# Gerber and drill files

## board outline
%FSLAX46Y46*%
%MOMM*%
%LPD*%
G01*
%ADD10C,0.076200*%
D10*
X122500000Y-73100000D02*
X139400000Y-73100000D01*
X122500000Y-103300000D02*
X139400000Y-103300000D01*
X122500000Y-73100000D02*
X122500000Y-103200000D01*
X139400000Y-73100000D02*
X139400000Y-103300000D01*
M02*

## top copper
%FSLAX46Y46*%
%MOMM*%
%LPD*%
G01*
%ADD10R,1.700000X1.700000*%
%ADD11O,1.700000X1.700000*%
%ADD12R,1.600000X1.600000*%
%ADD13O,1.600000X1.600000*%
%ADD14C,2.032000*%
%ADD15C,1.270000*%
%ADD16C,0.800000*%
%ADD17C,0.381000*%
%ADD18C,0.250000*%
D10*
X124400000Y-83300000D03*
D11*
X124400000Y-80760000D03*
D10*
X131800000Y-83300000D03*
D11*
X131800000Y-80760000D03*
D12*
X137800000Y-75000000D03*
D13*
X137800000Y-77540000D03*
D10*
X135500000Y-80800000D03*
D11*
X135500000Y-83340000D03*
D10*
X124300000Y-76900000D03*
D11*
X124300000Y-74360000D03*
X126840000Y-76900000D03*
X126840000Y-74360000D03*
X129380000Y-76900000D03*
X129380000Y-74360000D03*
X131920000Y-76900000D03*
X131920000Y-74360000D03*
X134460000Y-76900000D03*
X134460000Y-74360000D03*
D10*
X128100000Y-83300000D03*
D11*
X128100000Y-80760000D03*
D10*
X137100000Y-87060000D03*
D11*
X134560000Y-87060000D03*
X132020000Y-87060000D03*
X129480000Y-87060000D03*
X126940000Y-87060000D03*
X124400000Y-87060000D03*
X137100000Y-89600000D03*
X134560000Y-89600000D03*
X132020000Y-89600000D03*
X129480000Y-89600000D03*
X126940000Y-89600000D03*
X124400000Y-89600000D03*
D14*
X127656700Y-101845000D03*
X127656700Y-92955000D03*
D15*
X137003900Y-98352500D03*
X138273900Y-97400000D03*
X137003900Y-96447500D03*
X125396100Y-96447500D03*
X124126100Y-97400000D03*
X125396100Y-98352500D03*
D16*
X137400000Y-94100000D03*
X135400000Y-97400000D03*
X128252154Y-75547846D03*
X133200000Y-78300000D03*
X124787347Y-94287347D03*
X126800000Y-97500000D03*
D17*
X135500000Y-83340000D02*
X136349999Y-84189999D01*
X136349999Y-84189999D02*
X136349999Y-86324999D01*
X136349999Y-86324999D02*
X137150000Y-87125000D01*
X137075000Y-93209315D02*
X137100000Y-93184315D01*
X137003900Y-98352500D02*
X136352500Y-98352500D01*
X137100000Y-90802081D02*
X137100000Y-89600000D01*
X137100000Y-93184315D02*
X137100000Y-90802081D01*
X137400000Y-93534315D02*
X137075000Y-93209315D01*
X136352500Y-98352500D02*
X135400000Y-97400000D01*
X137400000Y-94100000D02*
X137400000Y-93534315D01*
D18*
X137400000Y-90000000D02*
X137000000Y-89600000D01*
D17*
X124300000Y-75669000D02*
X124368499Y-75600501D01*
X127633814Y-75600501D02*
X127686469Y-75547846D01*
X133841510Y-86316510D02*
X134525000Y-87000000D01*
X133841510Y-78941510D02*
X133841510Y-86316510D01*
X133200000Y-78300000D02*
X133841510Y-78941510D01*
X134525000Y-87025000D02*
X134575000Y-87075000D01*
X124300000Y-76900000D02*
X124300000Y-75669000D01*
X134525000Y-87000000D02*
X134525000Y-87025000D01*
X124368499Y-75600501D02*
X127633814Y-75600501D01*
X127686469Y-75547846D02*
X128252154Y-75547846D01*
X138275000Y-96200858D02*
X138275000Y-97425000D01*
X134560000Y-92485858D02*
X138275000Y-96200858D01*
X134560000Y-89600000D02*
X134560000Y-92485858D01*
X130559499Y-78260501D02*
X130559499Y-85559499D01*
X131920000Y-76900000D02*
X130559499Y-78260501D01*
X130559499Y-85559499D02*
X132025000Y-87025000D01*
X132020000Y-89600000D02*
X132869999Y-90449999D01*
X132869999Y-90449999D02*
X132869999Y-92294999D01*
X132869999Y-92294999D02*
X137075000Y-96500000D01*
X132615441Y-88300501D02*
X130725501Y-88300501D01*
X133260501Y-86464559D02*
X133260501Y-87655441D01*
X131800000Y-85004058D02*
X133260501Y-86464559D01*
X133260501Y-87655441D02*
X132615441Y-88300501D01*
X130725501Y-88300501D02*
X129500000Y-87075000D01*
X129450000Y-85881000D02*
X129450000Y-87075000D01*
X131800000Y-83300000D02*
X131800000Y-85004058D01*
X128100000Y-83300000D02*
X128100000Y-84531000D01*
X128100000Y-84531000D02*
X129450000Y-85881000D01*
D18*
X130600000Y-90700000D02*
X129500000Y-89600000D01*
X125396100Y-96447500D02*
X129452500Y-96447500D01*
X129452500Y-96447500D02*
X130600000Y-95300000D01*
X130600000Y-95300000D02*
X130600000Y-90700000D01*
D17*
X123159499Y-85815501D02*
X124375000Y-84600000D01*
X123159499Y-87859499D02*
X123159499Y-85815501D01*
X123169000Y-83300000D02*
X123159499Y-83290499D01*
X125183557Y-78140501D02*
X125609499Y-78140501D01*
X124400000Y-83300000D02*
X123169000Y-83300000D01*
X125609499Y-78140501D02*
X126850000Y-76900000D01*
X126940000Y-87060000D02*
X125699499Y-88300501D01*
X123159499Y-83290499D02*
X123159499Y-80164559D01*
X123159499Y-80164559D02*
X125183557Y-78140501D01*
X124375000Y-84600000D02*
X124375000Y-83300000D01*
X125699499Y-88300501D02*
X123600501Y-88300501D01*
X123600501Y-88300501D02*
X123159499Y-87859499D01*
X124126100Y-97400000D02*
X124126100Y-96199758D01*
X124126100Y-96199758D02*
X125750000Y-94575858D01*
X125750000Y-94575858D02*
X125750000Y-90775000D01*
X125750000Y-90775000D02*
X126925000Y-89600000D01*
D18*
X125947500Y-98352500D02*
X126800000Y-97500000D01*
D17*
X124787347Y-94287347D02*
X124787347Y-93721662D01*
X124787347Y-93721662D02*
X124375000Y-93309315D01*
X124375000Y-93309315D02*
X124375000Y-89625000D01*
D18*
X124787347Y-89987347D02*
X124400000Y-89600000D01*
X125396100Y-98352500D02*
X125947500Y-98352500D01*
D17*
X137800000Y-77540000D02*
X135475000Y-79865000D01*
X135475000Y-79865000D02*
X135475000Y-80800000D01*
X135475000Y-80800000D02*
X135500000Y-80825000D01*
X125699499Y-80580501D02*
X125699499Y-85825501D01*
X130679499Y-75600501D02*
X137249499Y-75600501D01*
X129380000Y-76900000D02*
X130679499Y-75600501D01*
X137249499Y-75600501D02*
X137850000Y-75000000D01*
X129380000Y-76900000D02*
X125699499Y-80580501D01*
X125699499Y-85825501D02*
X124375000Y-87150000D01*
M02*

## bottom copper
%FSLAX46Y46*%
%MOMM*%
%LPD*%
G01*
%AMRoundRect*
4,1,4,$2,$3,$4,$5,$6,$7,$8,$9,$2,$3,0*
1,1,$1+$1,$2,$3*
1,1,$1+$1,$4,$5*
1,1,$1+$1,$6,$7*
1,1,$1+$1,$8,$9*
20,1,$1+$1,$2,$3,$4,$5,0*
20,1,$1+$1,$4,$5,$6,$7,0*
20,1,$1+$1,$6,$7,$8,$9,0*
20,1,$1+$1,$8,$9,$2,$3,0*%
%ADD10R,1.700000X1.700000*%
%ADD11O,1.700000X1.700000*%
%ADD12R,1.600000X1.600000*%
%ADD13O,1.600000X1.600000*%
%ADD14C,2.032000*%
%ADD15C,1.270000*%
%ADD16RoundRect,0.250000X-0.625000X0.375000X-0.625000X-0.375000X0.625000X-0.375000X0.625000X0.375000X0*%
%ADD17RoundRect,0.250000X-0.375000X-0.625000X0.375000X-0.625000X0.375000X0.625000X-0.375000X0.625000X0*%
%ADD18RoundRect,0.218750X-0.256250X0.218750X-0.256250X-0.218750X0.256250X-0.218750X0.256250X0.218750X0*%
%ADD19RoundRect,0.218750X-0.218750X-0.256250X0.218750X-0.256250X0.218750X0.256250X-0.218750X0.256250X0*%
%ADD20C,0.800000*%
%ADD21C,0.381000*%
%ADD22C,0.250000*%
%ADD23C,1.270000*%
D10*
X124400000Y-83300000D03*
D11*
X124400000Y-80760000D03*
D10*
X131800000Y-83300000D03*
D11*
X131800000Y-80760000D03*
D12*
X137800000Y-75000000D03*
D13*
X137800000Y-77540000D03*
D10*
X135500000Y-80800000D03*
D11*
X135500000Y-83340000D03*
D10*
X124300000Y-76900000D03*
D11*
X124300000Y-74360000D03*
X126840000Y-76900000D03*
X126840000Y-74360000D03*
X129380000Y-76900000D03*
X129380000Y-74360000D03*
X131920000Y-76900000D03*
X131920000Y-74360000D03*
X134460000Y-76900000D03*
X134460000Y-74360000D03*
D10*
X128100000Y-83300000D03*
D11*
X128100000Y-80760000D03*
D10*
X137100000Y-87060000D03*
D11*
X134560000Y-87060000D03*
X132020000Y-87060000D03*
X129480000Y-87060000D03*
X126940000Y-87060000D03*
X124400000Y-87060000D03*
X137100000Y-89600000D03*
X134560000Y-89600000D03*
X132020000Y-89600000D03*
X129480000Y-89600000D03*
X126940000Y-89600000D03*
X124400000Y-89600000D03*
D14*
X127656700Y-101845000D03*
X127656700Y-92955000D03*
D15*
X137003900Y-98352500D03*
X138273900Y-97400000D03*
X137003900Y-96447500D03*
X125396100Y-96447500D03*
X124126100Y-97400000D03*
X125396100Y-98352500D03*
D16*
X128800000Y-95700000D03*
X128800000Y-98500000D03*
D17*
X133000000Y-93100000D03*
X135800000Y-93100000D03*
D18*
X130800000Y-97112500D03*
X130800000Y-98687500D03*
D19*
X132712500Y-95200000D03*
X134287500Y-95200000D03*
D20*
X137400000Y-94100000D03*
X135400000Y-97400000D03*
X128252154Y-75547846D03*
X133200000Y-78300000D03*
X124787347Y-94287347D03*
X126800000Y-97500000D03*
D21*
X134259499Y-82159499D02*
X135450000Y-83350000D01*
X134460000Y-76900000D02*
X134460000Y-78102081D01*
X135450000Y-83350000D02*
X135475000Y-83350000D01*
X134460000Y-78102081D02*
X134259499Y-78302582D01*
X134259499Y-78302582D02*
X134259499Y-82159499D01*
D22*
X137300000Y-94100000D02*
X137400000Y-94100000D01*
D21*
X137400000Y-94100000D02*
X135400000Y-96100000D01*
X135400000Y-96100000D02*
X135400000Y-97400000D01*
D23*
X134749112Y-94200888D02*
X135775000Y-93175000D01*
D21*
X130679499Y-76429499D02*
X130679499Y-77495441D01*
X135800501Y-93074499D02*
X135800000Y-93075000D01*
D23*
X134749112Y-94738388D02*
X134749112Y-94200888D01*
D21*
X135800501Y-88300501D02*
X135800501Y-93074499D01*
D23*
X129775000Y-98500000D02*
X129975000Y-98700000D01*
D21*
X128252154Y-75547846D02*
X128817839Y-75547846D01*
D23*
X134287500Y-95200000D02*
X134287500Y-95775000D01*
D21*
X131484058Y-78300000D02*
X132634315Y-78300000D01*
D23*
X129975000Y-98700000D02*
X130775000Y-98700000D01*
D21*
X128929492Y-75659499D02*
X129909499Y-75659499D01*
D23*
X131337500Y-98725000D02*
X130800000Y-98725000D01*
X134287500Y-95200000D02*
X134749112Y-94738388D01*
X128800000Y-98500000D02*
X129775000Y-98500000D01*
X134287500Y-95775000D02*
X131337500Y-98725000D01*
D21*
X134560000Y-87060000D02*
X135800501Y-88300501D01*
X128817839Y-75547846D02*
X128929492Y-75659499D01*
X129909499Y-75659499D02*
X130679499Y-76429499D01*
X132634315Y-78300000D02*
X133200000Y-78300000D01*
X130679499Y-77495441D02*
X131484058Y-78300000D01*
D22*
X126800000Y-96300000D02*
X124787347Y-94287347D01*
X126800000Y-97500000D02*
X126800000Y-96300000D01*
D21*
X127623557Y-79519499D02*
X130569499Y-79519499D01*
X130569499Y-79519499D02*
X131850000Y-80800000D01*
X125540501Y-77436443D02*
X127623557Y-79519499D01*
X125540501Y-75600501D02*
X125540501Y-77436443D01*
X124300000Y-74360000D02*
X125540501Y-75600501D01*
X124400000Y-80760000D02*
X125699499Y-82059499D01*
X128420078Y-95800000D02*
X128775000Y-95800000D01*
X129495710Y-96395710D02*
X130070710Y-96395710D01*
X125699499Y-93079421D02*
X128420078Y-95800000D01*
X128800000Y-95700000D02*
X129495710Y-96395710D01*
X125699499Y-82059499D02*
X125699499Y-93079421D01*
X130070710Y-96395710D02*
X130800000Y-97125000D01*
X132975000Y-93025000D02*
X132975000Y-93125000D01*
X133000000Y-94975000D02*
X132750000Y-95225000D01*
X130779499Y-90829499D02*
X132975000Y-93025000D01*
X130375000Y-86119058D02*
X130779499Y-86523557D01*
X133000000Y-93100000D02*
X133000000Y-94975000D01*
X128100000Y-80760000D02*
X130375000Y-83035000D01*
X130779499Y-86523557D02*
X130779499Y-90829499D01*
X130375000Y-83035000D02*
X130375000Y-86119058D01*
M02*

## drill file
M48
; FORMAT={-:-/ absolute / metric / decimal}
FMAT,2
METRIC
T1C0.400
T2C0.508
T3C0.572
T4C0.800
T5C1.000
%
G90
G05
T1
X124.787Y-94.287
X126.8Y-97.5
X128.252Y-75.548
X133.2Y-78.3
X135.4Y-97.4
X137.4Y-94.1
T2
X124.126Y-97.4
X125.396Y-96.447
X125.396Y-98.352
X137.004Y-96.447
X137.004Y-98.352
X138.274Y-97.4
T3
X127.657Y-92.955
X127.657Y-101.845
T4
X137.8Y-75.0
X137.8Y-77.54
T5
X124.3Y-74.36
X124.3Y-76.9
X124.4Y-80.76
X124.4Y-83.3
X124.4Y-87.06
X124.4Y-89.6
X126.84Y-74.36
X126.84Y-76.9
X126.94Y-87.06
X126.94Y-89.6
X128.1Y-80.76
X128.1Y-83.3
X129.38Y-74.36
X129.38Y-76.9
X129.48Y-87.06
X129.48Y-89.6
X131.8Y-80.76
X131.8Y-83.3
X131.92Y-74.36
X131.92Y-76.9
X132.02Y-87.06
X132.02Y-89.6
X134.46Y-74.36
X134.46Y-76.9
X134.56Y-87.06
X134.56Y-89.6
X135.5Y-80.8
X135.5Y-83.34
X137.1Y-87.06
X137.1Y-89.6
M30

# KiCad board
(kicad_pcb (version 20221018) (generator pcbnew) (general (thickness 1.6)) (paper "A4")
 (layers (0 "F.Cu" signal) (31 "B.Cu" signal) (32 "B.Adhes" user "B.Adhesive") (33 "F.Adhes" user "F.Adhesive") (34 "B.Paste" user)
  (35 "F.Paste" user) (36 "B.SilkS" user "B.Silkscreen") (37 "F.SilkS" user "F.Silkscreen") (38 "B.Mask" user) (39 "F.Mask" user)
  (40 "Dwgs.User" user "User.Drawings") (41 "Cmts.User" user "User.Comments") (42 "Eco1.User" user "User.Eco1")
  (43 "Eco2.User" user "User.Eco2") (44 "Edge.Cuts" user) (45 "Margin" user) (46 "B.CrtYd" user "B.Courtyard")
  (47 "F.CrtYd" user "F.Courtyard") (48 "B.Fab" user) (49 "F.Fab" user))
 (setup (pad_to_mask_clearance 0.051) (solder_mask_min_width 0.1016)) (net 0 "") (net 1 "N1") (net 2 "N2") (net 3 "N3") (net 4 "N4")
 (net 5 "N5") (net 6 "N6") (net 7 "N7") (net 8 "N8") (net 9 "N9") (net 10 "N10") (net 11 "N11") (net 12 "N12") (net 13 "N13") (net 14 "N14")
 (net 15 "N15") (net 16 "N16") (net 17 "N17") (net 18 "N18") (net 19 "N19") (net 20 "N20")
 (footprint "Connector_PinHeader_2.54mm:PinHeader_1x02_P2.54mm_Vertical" (layer "F.Cu") (at 124.4 83.3 180)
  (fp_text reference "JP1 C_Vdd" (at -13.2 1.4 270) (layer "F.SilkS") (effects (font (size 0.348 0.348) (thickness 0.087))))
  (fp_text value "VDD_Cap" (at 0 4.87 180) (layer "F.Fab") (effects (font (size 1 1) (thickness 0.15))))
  (pad "1" thru_hole rect (at 0 0 180) (size 1.7 1.7) (drill 1) (layers "*.Cu" "*.Mask") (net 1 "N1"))
  (pad "2" thru_hole oval (at 0 2.54 180) (size 1.7 1.7) (drill 1) (layers "*.Cu" "*.Mask") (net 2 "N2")))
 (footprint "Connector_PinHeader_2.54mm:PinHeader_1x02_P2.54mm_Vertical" (layer "F.Cu") (at 131.8 83.3 180)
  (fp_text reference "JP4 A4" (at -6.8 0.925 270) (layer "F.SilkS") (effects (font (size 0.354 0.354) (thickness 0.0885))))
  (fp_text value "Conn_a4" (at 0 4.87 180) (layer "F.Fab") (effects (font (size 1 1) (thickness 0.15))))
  (pad "1" thru_hole rect (at 0 0 180) (size 1.7 1.7) (drill 1) (layers "*.Cu" "*.Mask") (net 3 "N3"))
  (pad "2" thru_hole oval (at 0 2.54 180) (size 1.7 1.7) (drill 1) (layers "*.Cu" "*.Mask") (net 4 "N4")))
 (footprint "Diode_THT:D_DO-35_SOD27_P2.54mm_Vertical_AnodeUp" (layer "F.Cu") (at 137.8 75 -90)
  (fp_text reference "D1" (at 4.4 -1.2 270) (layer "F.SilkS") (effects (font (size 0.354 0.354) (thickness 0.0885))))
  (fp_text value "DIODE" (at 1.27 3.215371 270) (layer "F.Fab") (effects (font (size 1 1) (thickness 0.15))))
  (pad "1" thru_hole rect (at 0 0 270) (size 1.6 1.6) (drill 0.8) (layers "*.Cu" "*.Mask") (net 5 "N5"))
  (pad "2" thru_hole oval (at 2.54 0 270) (size 1.6 1.6) (drill 0.8) (layers "*.Cu" "*.Mask") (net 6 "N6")))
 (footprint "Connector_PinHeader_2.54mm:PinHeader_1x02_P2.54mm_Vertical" (layer "F.Cu") (at 135.5 80.8)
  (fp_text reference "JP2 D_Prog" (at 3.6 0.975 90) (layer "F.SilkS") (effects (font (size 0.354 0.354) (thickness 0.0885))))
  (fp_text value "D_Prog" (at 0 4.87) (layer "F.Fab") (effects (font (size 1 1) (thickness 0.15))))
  (pad "1" thru_hole rect (at 0 0) (size 1.7 1.7) (drill 1) (layers "*.Cu" "*.Mask") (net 6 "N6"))
  (pad "2" thru_hole oval (at 0 2.54) (size 1.7 1.7) (drill 1) (layers "*.Cu" "*.Mask") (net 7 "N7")))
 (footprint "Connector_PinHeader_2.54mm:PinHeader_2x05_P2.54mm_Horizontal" (layer "F.Cu") (at 124.3 76.9 90)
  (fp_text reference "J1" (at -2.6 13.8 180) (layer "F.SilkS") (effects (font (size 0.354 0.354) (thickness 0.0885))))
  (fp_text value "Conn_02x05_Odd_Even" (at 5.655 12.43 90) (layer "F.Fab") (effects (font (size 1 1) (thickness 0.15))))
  (pad "1" thru_hole rect (at 0 0 90) (size 1.7 1.7) (drill 1) (layers "*.Cu" "*.Mask") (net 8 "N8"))
  (pad "2" thru_hole oval (at 2.54 0 90) (size 1.7 1.7) (drill 1) (layers "*.Cu" "*.Mask") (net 4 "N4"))
  (pad "3" thru_hole oval (at 0 2.54 90) (size 1.7 1.7) (drill 1) (layers "*.Cu" "*.Mask") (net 1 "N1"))
  (pad "4" thru_hole oval (at 2.54 2.54 90) (size 1.7 1.7) (drill 1) (layers "*.Cu" "*.Mask") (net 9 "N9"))
  (pad "5" thru_hole oval (at 0 5.08 90) (size 1.7 1.7) (drill 1) (layers "*.Cu" "*.Mask") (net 5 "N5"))
  (pad "6" thru_hole oval (at 2.54 5.08 90) (size 1.7 1.7) (drill 1) (layers "*.Cu" "*.Mask") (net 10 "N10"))
  (pad "7" thru_hole oval (at 0 7.62 90) (size 1.7 1.7) (drill 1) (layers "*.Cu" "*.Mask") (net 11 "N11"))
  (pad "8" thru_hole oval (at 2.54 7.62 90) (size 1.7 1.7) (drill 1) (layers "*.Cu" "*.Mask") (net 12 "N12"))
  (pad "9" thru_hole oval (at 0 10.16 90) (size 1.7 1.7) (drill 1) (layers "*.Cu" "*.Mask") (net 7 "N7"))
  (pad "10" thru_hole oval (at 2.54 10.16 90) (size 1.7 1.7) (drill 1) (layers "*.Cu" "*.Mask") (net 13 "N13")))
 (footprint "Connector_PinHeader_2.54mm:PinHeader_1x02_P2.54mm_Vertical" (layer "F.Cu") (at 128.1 83.3 180)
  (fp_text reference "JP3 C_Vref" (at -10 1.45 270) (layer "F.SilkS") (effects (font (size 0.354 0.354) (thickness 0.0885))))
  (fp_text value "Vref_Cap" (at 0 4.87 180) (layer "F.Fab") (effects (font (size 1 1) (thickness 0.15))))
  (pad "1" thru_hole rect (at 0 0 180) (size 1.7 1.7) (drill 1) (layers "*.Cu" "*.Mask") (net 3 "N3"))
  (pad "2" thru_hole oval (at 0 2.54 180) (size 1.7 1.7) (drill 1) (layers "*.Cu" "*.Mask") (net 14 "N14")))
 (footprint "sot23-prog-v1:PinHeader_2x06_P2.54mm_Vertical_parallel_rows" (layer "F.Cu") (at 137.1 87.06 -90)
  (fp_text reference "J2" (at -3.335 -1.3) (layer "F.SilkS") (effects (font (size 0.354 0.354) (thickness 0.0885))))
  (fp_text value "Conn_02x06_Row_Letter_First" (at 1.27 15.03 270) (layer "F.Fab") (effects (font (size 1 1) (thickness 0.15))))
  (pad "a1" thru_hole rect (at 0 0 270) (size 1.7 1.7) (drill 1) (layers "*.Cu" "*.Mask") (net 7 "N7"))
  (pad "a2" thru_hole oval (at 0 2.54 270) (size 1.7 1.7) (drill 1) (layers "*.Cu" "*.Mask") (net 8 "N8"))
  (pad "a3" thru_hole oval (at 0 5.08 270) (size 1.7 1.7) (drill 1) (layers "*.Cu" "*.Mask") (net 11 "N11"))
  (pad "a4" thru_hole oval (at 0 7.62 270) (size 1.7 1.7) (drill 1) (layers "*.Cu" "*.Mask") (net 3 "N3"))
  (pad "a5" thru_hole oval (at 0 10.16 270) (size 1.7 1.7) (drill 1) (layers "*.Cu" "*.Mask") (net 1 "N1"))
  (pad "a6" thru_hole oval (at 0 12.7 270) (size 1.7 1.7) (drill 1) (layers "*.Cu" "*.Mask") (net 5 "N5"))
  (pad "b1" thru_hole oval (at 2.54 0 270) (size 1.7 1.7) (drill 1) (layers "*.Cu" "*.Mask") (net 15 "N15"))
  (pad "b2" thru_hole oval (at 2.54 2.54 270) (size 1.7 1.7) (drill 1) (layers "*.Cu" "*.Mask") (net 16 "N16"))
  (pad "b3" thru_hole oval (at 2.54 5.08 270) (size 1.7 1.7) (drill 1) (layers "*.Cu" "*.Mask") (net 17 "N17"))
  (pad "b4" thru_hole oval (at 2.54 7.62 270) (size 1.7 1.7) (drill 1) (layers "*.Cu" "*.Mask") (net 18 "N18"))
  (pad "b5" thru_hole oval (at 2.54 10.16 270) (size 1.7 1.7) (drill 1) (layers "*.Cu" "*.Mask") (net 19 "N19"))
  (pad "b6" thru_hole oval (at 2.54 12.7 270) (size 1.7 1.7) (drill 1) (layers "*.Cu" "*.Mask") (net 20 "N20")))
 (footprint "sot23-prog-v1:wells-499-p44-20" (layer "F.Cu") (at 131.2 97.4 90)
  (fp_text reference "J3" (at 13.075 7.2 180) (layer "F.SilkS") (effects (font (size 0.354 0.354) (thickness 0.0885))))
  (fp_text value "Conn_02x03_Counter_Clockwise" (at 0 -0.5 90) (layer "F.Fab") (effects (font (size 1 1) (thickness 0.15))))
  (pad "" thru_hole circle (at -4.445 -3.5433 90) (size 2.032 2.032) (drill 0.5715) (layers "*.Cu" "*.Mask"))
  (pad "" thru_hole circle (at 4.445 -3.5433 90) (size 2.032 2.032) (drill 0.5715) (layers "*.Cu" "*.Mask"))
  (pad "1" thru_hole circle (at -0.9525 5.8039 90) (size 1.27 1.27) (drill 0.508) (layers "*.Cu" "*.Mask") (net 15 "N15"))
  (pad "2" thru_hole circle (at 0 7.0739 90) (size 1.27 1.27) (drill 0.508) (layers "*.Cu" "*.Mask") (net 16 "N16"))
  (pad "3" thru_hole circle (at 0.9525 5.8039 90) (size 1.27 1.27) (drill 0.508) (layers "*.Cu" "*.Mask") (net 17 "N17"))
  (pad "4" thru_hole circle (at 0.9525 -5.8039 90) (size 1.27 1.27) (drill 0.508) (layers "*.Cu" "*.Mask") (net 18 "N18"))
  (pad "5" thru_hole circle (at 0 -7.0739 90) (size 1.27 1.27) (drill 0.508) (layers "*.Cu" "*.Mask") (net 19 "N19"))
  (pad "6" thru_hole circle (at -0.9525 -5.8039 90) (size 1.27 1.27) (drill 0.508) (layers "*.Cu" "*.Mask") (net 20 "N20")))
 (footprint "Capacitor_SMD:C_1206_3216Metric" (layer "B.Cu") (at 128.8 97.1 -90)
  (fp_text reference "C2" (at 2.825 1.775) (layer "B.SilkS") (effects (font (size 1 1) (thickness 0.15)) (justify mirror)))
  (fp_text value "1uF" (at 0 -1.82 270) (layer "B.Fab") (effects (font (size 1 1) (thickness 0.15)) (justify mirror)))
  (pad "1" smd roundrect (at -1.4 0 270) (size 1.25 1.75) (layers "B.Cu" "B.Paste" "B.Mask") (roundrect_rratio 0.2) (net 2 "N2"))
  (pad "2" smd roundrect (at 1.4 0 270) (size 1.25 1.75) (layers "B.Cu" "B.Paste" "B.Mask") (roundrect_rratio 0.2) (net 8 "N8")))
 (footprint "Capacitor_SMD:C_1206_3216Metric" (layer "B.Cu") (at 134.4 93.1)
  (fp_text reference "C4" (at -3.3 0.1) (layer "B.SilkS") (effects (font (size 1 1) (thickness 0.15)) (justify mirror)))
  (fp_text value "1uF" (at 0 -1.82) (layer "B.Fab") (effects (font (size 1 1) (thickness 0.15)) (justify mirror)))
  (pad "1" smd roundrect (at -1.4 0) (size 1.25 1.75) (layers "B.Cu" "B.Paste" "B.Mask") (roundrect_rratio 0.2) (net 14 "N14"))
  (pad "2" smd roundrect (at 1.4 0) (size 1.25 1.75) (layers "B.Cu" "B.Paste" "B.Mask") (roundrect_rratio 0.2) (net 8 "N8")))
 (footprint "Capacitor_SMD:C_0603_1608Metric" (layer "B.Cu") (at 130.8 97.9 -90)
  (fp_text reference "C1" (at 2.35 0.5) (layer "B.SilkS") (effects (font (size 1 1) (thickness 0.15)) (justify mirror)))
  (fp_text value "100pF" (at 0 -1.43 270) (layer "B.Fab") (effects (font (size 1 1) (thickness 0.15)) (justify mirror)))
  (pad "1" smd roundrect (at -0.7875 0 270) (size 0.875 0.95) (layers "B.Cu" "B.Paste" "B.Mask") (roundrect_rratio 0.25) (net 2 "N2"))
  (pad "2" smd roundrect (at 0.7875 0 270) (size 0.875 0.95) (layers "B.Cu" "B.Paste" "B.Mask") (roundrect_rratio 0.25) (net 8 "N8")))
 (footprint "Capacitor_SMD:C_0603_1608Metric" (layer "B.Cu") (at 133.5 95.2)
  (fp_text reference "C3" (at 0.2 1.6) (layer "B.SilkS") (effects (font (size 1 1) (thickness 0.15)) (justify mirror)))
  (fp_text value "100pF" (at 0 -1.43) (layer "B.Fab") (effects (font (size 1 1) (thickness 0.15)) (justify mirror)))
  (pad "1" smd roundrect (at -0.7875 0) (size 0.875 0.95) (layers "B.Cu" "B.Paste" "B.Mask") (roundrect_rratio 0.25) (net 14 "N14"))
  (pad "2" smd roundrect (at 0.7875 0) (size 0.875 0.95) (layers "B.Cu" "B.Paste" "B.Mask") (roundrect_rratio 0.25) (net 8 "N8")))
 (gr_line (start 122.5 73.1) (end 139.4 73.1) (stroke (width 0.0762) (type solid)) (layer "Edge.Cuts"))
 (gr_line (start 122.5 103.3) (end 139.4 103.3) (stroke (width 0.0762) (type solid)) (layer "Edge.Cuts"))
 (gr_line (start 122.5 73.1) (end 122.5 103.2) (stroke (width 0.0762) (type solid)) (layer "Edge.Cuts"))
 (gr_line (start 139.4 73.1) (end 139.4 103.3) (stroke (width 0.0762) (type solid)) (layer "Edge.Cuts"))
 (segment (start 135.5 83.34) (end 136.349999 84.189999) (width 0.381) (layer "F.Cu") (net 7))
 (segment (start 136.349999 84.189999) (end 136.349999 86.324999) (width 0.381) (layer "F.Cu") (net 7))
 (segment (start 136.349999 86.324999) (end 137.15 87.125) (width 0.381) (layer "F.Cu") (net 7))
 (segment (start 134.259499 82.159499) (end 135.45 83.35) (width 0.381) (layer "B.Cu") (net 7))
 (segment (start 134.46 76.9) (end 134.46 78.102081) (width 0.381) (layer "B.Cu") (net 7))
 (segment (start 135.45 83.35) (end 135.475 83.35) (width 0.381) (layer "B.Cu") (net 7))
 (segment (start 134.46 78.102081) (end 134.259499 78.302582) (width 0.381) (layer "B.Cu") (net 7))
 (segment (start 134.259499 78.302582) (end 134.259499 82.159499) (width 0.381) (layer "B.Cu") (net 7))
 (segment (start 137.075 93.209315) (end 137.1 93.184315) (width 0.381) (layer "F.Cu") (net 15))
 (segment (start 137.0039 98.3525) (end 136.3525 98.3525) (width 0.381) (layer "F.Cu") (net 15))
 (segment (start 137.1 90.802081) (end 137.1 89.6) (width 0.381) (layer "F.Cu") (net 15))
 (segment (start 137.1 93.184315) (end 137.1 90.802081) (width 0.381) (layer "F.Cu") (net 15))
 (segment (start 137.4 93.534315) (end 137.075 93.209315) (width 0.381) (layer "F.Cu") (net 15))
 (segment (start 136.3525 98.3525) (end 135.4 97.4) (width 0.381) (layer "F.Cu") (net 15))
 (segment (start 137.4 94.1) (end 137.4 93.534315) (width 0.381) (layer "F.Cu") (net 15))
 (segment (start 137.4 90) (end 137 89.6) (width 0.25) (layer "F.Cu") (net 15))
 (via (at 137.4 94.1) (size 0.8) (drill 0.4) (layers "F.Cu" "B.Cu") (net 15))
 (via (at 135.4 97.4) (size 0.8) (drill 0.4) (layers "F.Cu" "B.Cu") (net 15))
 (segment (start 137.3 94.1) (end 137.4 94.1) (width 0.25) (layer "B.Cu") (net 15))
 (segment (start 137.4 94.1) (end 135.4 96.1) (width 0.381) (layer "B.Cu") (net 15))
 (segment (start 135.4 96.1) (end 135.4 97.4) (width 0.381) (layer "B.Cu") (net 15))
 (segment (start 124.3 75.669) (end 124.368499 75.600501) (width 0.381) (layer "F.Cu") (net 8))
 (segment (start 127.633814 75.600501) (end 127.686469 75.547846) (width 0.381) (layer "F.Cu") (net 8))
 (segment (start 133.84151 86.31651) (end 134.525 87) (width 0.381) (layer "F.Cu") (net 8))
 (segment (start 133.84151 78.94151) (end 133.84151 86.31651) (width 0.381) (layer "F.Cu") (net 8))
 (segment (start 133.2 78.3) (end 133.84151 78.94151) (width 0.381) (layer "F.Cu") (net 8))
 (segment (start 134.525 87.025) (end 134.575 87.075) (width 0.381) (layer "F.Cu") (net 8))
 (segment (start 124.3 76.9) (end 124.3 75.669) (width 0.381) (layer "F.Cu") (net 8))
 (segment (start 134.525 87) (end 134.525 87.025) (width 0.381) (layer "F.Cu") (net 8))
 (segment (start 124.368499 75.600501) (end 127.633814 75.600501) (width 0.381) (layer "F.Cu") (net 8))
 (segment (start 127.686469 75.547846) (end 128.252154 75.547846) (width 0.381) (layer "F.Cu") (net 8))
 (via (at 128.252154 75.547846) (size 0.8) (drill 0.4) (layers "F.Cu" "B.Cu") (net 8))
 (via (at 133.2 78.3) (size 0.8) (drill 0.4) (layers "F.Cu" "B.Cu") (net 8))
 (segment (start 134.749112 94.200888) (end 135.775 93.175) (width 1.27) (layer "B.Cu") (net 8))
 (segment (start 130.679499 76.429499) (end 130.679499 77.495441) (width 0.381) (layer "B.Cu") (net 8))
 (segment (start 135.800501 93.074499) (end 135.8 93.075) (width 0.381) (layer "B.Cu") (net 8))
 (segment (start 134.749112 94.738388) (end 134.749112 94.200888) (width 1.27) (layer "B.Cu") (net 8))
 (segment (start 135.800501 88.300501) (end 135.800501 93.074499) (width 0.381) (layer "B.Cu") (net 8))
 (segment (start 129.775 98.5) (end 129.975 98.7) (width 1.27) (layer "B.Cu") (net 8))
 (segment (start 128.252154 75.547846) (end 128.817839 75.547846) (width 0.381) (layer "B.Cu") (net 8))
 (segment (start 134.2875 95.2) (end 134.2875 95.775) (width 1.27) (layer "B.Cu") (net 8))
 (segment (start 131.484058 78.3) (end 132.634315 78.3) (width 0.381) (layer "B.Cu") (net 8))
 (segment (start 129.975 98.7) (end 130.775 98.7) (width 1.27) (layer "B.Cu") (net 8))
 (segment (start 128.929492 75.659499) (end 129.909499 75.659499) (width 0.381) (layer "B.Cu") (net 8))
 (segment (start 131.3375 98.725) (end 130.8 98.725) (width 1.27) (layer "B.Cu") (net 8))
 (segment (start 134.2875 95.2) (end 134.749112 94.738388) (width 1.27) (layer "B.Cu") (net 8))
 (segment (start 128.8 98.5) (end 129.775 98.5) (width 1.27) (layer "B.Cu") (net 8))
 (segment (start 134.2875 95.775) (end 131.3375 98.725) (width 1.27) (layer "B.Cu") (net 8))
 (segment (start 134.56 87.06) (end 135.800501 88.300501) (width 0.381) (layer "B.Cu") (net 8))
 (segment (start 128.817839 75.547846) (end 128.929492 75.659499) (width 0.381) (layer "B.Cu") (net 8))
 (segment (start 129.909499 75.659499) (end 130.679499 76.429499) (width 0.381) (layer "B.Cu") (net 8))
 (segment (start 132.634315 78.3) (end 133.2 78.3) (width 0.381) (layer "B.Cu") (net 8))
 (segment (start 130.679499 77.495441) (end 131.484058 78.3) (width 0.381) (layer "B.Cu") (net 8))
 (segment (start 138.275 96.200858) (end 138.275 97.425) (width 0.381) (layer "F.Cu") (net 16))
 (segment (start 134.56 92.485858) (end 138.275 96.200858) (width 0.381) (layer "F.Cu") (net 16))
 (segment (start 134.56 89.6) (end 134.56 92.485858) (width 0.381) (layer "F.Cu") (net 16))
 (segment (start 130.559499 78.260501) (end 130.559499 85.559499) (width 0.381) (layer "F.Cu") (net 11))
 (segment (start 131.92 76.9) (end 130.559499 78.260501) (width 0.381) (layer "F.Cu") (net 11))
 (segment (start 130.559499 85.559499) (end 132.025 87.025) (width 0.381) (layer "F.Cu") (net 11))
 (segment (start 132.02 89.6) (end 132.869999 90.449999) (width 0.381) (layer "F.Cu") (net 17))
 (segment (start 132.869999 90.449999) (end 132.869999 92.294999) (width 0.381) (layer "F.Cu") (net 17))
 (segment (start 132.869999 92.294999) (end 137.075 96.5) (width 0.381) (layer "F.Cu") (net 17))
 (segment (start 132.615441 88.300501) (end 130.725501 88.300501) (width 0.381) (layer "F.Cu") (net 3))
 (segment (start 133.260501 86.464559) (end 133.260501 87.655441) (width 0.381) (layer "F.Cu") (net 3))
 (segment (start 131.8 85.004058) (end 133.260501 86.464559) (width 0.381) (layer "F.Cu") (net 3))
 (segment (start 133.260501 87.655441) (end 132.615441 88.300501) (width 0.381) (layer "F.Cu") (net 3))
 (segment (start 130.725501 88.300501) (end 129.5 87.075) (width 0.381) (layer "F.Cu") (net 3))
 (segment (start 129.45 85.881) (end 129.45 87.075) (width 0.381) (layer "F.Cu") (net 3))
 (segment (start 131.8 83.3) (end 131.8 85.004058) (width 0.381) (layer "F.Cu") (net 3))
 (segment (start 128.1 83.3) (end 128.1 84.531) (width 0.381) (layer "F.Cu") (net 3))
 (segment (start 128.1 84.531) (end 129.45 85.881) (width 0.381) (layer "F.Cu") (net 3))
 (segment (start 130.6 90.7) (end 129.5 89.6) (width 0.25) (layer "F.Cu") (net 18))
 (segment (start 125.3961 96.4475) (end 129.4525 96.4475) (width 0.25) (layer "F.Cu") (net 18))
 (segment (start 129.4525 96.4475) (end 130.6 95.3) (width 0.25) (layer "F.Cu") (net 18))
 (segment (start 130.6 95.3) (end 130.6 90.7) (width 0.25) (layer "F.Cu") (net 18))
 (segment (start 123.159499 85.815501) (end 124.375 84.6) (width 0.381) (layer "F.Cu") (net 1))
 (segment (start 123.159499 87.859499) (end 123.159499 85.815501) (width 0.381) (layer "F.Cu") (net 1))
 (segment (start 123.169 83.3) (end 123.159499 83.290499) (width 0.381) (layer "F.Cu") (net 1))
 (segment (start 125.183557 78.140501) (end 125.609499 78.140501) (width 0.381) (layer "F.Cu") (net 1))
 (segment (start 124.4 83.3) (end 123.169 83.3) (width 0.381) (layer "F.Cu") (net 1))
 (segment (start 125.609499 78.140501) (end 126.85 76.9) (width 0.381) (layer "F.Cu") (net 1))
 (segment (start 126.94 87.06) (end 125.699499 88.300501) (width 0.381) (layer "F.Cu") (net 1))
 (segment (start 123.159499 83.290499) (end 123.159499 80.164559) (width 0.381) (layer "F.Cu") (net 1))
 (segment (start 123.159499 80.164559) (end 125.183557 78.140501) (width 0.381) (layer "F.Cu") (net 1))
 (segment (start 124.375 84.6) (end 124.375 83.3) (width 0.381) (layer "F.Cu") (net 1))
 (segment (start 125.699499 88.300501) (end 123.600501 88.300501) (width 0.381) (layer "F.Cu") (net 1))
 (segment (start 123.600501 88.300501) (end 123.159499 87.859499) (width 0.381) (layer "F.Cu") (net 1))
 (segment (start 124.1261 97.4) (end 124.1261 96.199758) (width 0.381) (layer "F.Cu") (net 19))
 (segment (start 124.1261 96.199758) (end 125.75 94.575858) (width 0.381) (layer "F.Cu") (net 19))
 (segment (start 125.75 94.575858) (end 125.75 90.775) (width 0.381) (layer "F.Cu") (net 19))
 (segment (start 125.75 90.775) (end 126.925 89.6) (width 0.381) (layer "F.Cu") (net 19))
 (segment (start 125.9475 98.3525) (end 126.8 97.5) (width 0.25) (layer "F.Cu") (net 20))
 (segment (start 124.787347 94.287347) (end 124.787347 93.721662) (width 0.381) (layer "F.Cu") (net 20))
 (segment (start 124.787347 93.721662) (end 124.375 93.309315) (width 0.381) (layer "F.Cu") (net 20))
 (segment (start 124.375 93.309315) (end 124.375 89.625) (width 0.381) (layer "F.Cu") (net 20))
 (segment (start 124.787347 89.987347) (end 124.4 89.6) (width 0.25) (layer "F.Cu") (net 20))
 (segment (start 125.3961 98.3525) (end 125.9475 98.3525) (width 0.25) (layer "F.Cu") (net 20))
 (via (at 124.787347 94.287347) (size 0.8) (drill 0.4) (layers "F.Cu" "B.Cu") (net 20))
 (via (at 126.8 97.5) (size 0.8) (drill 0.4) (layers "F.Cu" "B.Cu") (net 20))
 (segment (start 126.8 96.3) (end 124.787347 94.287347) (width 0.25) (layer "B.Cu") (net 20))
 (segment (start 126.8 97.5) (end 126.8 96.3) (width 0.25) (layer "B.Cu") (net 20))
 (segment (start 137.8 77.54) (end 135.475 79.865) (width 0.381) (layer "F.Cu") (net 6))
 (segment (start 135.475 79.865) (end 135.475 80.8) (width 0.381) (layer "F.Cu") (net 6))
 (segment (start 135.475 80.8) (end 135.5 80.825) (width 0.381) (layer "F.Cu") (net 6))
 (segment (start 125.699499 80.580501) (end 125.699499 85.825501) (width 0.381) (layer "F.Cu") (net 5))
 (segment (start 130.679499 75.600501) (end 137.249499 75.600501) (width 0.381) (layer "F.Cu") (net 5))
 (segment (start 129.38 76.9) (end 130.679499 75.600501) (width 0.381) (layer "F.Cu") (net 5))
 (segment (start 137.249499 75.600501) (end 137.85 75) (width 0.381) (layer "F.Cu") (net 5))
 (segment (start 129.38 76.9) (end 125.699499 80.580501) (width 0.381) (layer "F.Cu") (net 5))
 (segment (start 125.699499 85.825501) (end 124.375 87.15) (width 0.381) (layer "F.Cu") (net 5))
 (segment (start 127.623557 79.519499) (end 130.569499 79.519499) (width 0.381) (layer "B.Cu") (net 4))
 (segment (start 130.569499 79.519499) (end 131.85 80.8) (width 0.381) (layer "B.Cu") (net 4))
 (segment (start 125.540501 77.436443) (end 127.623557 79.519499) (width 0.381) (layer "B.Cu") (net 4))
 (segment (start 125.540501 75.600501) (end 125.540501 77.436443) (width 0.381) (layer "B.Cu") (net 4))
 (segment (start 124.3 74.36) (end 125.540501 75.600501) (width 0.381) (layer "B.Cu") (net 4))
 (segment (start 124.4 80.76) (end 125.699499 82.059499) (width 0.381) (layer "B.Cu") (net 2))
 (segment (start 128.420078 95.8) (end 128.775 95.8) (width 0.381) (layer "B.Cu") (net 2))
 (segment (start 129.49571 96.39571) (end 130.07071 96.39571) (width 0.381) (layer "B.Cu") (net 2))
 (segment (start 125.699499 93.079421) (end 128.420078 95.8) (width 0.381) (layer "B.Cu") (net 2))
 (segment (start 128.8 95.7) (end 129.49571 96.39571) (width 0.381) (layer "B.Cu") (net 2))
 (segment (start 125.699499 82.059499) (end 125.699499 93.079421) (width 0.381) (layer "B.Cu") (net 2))
 (segment (start 130.07071 96.39571) (end 130.8 97.125) (width 0.381) (layer "B.Cu") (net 2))
 (segment (start 132.975 93.025) (end 132.975 93.125) (width 0.381) (layer "B.Cu") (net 14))
 (segment (start 133 94.975) (end 132.75 95.225) (width 0.381) (layer "B.Cu") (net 14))
 (segment (start 130.779499 90.829499) (end 132.975 93.025) (width 0.381) (layer "B.Cu") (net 14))
 (segment (start 130.375 86.119058) (end 130.779499 86.523557) (width 0.381) (layer "B.Cu") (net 14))
 (segment (start 133 93.1) (end 133 94.975) (width 0.381) (layer "B.Cu") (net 14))
 (segment (start 128.1 80.76) (end 130.375 83.035) (width 0.381) (layer "B.Cu") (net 14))
 (segment (start 130.779499 86.523557) (end 130.779499 90.829499) (width 0.381) (layer "B.Cu") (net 14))
 (segment (start 130.375 83.035) (end 130.375 86.119058) (width 0.381) (layer "B.Cu") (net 14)))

